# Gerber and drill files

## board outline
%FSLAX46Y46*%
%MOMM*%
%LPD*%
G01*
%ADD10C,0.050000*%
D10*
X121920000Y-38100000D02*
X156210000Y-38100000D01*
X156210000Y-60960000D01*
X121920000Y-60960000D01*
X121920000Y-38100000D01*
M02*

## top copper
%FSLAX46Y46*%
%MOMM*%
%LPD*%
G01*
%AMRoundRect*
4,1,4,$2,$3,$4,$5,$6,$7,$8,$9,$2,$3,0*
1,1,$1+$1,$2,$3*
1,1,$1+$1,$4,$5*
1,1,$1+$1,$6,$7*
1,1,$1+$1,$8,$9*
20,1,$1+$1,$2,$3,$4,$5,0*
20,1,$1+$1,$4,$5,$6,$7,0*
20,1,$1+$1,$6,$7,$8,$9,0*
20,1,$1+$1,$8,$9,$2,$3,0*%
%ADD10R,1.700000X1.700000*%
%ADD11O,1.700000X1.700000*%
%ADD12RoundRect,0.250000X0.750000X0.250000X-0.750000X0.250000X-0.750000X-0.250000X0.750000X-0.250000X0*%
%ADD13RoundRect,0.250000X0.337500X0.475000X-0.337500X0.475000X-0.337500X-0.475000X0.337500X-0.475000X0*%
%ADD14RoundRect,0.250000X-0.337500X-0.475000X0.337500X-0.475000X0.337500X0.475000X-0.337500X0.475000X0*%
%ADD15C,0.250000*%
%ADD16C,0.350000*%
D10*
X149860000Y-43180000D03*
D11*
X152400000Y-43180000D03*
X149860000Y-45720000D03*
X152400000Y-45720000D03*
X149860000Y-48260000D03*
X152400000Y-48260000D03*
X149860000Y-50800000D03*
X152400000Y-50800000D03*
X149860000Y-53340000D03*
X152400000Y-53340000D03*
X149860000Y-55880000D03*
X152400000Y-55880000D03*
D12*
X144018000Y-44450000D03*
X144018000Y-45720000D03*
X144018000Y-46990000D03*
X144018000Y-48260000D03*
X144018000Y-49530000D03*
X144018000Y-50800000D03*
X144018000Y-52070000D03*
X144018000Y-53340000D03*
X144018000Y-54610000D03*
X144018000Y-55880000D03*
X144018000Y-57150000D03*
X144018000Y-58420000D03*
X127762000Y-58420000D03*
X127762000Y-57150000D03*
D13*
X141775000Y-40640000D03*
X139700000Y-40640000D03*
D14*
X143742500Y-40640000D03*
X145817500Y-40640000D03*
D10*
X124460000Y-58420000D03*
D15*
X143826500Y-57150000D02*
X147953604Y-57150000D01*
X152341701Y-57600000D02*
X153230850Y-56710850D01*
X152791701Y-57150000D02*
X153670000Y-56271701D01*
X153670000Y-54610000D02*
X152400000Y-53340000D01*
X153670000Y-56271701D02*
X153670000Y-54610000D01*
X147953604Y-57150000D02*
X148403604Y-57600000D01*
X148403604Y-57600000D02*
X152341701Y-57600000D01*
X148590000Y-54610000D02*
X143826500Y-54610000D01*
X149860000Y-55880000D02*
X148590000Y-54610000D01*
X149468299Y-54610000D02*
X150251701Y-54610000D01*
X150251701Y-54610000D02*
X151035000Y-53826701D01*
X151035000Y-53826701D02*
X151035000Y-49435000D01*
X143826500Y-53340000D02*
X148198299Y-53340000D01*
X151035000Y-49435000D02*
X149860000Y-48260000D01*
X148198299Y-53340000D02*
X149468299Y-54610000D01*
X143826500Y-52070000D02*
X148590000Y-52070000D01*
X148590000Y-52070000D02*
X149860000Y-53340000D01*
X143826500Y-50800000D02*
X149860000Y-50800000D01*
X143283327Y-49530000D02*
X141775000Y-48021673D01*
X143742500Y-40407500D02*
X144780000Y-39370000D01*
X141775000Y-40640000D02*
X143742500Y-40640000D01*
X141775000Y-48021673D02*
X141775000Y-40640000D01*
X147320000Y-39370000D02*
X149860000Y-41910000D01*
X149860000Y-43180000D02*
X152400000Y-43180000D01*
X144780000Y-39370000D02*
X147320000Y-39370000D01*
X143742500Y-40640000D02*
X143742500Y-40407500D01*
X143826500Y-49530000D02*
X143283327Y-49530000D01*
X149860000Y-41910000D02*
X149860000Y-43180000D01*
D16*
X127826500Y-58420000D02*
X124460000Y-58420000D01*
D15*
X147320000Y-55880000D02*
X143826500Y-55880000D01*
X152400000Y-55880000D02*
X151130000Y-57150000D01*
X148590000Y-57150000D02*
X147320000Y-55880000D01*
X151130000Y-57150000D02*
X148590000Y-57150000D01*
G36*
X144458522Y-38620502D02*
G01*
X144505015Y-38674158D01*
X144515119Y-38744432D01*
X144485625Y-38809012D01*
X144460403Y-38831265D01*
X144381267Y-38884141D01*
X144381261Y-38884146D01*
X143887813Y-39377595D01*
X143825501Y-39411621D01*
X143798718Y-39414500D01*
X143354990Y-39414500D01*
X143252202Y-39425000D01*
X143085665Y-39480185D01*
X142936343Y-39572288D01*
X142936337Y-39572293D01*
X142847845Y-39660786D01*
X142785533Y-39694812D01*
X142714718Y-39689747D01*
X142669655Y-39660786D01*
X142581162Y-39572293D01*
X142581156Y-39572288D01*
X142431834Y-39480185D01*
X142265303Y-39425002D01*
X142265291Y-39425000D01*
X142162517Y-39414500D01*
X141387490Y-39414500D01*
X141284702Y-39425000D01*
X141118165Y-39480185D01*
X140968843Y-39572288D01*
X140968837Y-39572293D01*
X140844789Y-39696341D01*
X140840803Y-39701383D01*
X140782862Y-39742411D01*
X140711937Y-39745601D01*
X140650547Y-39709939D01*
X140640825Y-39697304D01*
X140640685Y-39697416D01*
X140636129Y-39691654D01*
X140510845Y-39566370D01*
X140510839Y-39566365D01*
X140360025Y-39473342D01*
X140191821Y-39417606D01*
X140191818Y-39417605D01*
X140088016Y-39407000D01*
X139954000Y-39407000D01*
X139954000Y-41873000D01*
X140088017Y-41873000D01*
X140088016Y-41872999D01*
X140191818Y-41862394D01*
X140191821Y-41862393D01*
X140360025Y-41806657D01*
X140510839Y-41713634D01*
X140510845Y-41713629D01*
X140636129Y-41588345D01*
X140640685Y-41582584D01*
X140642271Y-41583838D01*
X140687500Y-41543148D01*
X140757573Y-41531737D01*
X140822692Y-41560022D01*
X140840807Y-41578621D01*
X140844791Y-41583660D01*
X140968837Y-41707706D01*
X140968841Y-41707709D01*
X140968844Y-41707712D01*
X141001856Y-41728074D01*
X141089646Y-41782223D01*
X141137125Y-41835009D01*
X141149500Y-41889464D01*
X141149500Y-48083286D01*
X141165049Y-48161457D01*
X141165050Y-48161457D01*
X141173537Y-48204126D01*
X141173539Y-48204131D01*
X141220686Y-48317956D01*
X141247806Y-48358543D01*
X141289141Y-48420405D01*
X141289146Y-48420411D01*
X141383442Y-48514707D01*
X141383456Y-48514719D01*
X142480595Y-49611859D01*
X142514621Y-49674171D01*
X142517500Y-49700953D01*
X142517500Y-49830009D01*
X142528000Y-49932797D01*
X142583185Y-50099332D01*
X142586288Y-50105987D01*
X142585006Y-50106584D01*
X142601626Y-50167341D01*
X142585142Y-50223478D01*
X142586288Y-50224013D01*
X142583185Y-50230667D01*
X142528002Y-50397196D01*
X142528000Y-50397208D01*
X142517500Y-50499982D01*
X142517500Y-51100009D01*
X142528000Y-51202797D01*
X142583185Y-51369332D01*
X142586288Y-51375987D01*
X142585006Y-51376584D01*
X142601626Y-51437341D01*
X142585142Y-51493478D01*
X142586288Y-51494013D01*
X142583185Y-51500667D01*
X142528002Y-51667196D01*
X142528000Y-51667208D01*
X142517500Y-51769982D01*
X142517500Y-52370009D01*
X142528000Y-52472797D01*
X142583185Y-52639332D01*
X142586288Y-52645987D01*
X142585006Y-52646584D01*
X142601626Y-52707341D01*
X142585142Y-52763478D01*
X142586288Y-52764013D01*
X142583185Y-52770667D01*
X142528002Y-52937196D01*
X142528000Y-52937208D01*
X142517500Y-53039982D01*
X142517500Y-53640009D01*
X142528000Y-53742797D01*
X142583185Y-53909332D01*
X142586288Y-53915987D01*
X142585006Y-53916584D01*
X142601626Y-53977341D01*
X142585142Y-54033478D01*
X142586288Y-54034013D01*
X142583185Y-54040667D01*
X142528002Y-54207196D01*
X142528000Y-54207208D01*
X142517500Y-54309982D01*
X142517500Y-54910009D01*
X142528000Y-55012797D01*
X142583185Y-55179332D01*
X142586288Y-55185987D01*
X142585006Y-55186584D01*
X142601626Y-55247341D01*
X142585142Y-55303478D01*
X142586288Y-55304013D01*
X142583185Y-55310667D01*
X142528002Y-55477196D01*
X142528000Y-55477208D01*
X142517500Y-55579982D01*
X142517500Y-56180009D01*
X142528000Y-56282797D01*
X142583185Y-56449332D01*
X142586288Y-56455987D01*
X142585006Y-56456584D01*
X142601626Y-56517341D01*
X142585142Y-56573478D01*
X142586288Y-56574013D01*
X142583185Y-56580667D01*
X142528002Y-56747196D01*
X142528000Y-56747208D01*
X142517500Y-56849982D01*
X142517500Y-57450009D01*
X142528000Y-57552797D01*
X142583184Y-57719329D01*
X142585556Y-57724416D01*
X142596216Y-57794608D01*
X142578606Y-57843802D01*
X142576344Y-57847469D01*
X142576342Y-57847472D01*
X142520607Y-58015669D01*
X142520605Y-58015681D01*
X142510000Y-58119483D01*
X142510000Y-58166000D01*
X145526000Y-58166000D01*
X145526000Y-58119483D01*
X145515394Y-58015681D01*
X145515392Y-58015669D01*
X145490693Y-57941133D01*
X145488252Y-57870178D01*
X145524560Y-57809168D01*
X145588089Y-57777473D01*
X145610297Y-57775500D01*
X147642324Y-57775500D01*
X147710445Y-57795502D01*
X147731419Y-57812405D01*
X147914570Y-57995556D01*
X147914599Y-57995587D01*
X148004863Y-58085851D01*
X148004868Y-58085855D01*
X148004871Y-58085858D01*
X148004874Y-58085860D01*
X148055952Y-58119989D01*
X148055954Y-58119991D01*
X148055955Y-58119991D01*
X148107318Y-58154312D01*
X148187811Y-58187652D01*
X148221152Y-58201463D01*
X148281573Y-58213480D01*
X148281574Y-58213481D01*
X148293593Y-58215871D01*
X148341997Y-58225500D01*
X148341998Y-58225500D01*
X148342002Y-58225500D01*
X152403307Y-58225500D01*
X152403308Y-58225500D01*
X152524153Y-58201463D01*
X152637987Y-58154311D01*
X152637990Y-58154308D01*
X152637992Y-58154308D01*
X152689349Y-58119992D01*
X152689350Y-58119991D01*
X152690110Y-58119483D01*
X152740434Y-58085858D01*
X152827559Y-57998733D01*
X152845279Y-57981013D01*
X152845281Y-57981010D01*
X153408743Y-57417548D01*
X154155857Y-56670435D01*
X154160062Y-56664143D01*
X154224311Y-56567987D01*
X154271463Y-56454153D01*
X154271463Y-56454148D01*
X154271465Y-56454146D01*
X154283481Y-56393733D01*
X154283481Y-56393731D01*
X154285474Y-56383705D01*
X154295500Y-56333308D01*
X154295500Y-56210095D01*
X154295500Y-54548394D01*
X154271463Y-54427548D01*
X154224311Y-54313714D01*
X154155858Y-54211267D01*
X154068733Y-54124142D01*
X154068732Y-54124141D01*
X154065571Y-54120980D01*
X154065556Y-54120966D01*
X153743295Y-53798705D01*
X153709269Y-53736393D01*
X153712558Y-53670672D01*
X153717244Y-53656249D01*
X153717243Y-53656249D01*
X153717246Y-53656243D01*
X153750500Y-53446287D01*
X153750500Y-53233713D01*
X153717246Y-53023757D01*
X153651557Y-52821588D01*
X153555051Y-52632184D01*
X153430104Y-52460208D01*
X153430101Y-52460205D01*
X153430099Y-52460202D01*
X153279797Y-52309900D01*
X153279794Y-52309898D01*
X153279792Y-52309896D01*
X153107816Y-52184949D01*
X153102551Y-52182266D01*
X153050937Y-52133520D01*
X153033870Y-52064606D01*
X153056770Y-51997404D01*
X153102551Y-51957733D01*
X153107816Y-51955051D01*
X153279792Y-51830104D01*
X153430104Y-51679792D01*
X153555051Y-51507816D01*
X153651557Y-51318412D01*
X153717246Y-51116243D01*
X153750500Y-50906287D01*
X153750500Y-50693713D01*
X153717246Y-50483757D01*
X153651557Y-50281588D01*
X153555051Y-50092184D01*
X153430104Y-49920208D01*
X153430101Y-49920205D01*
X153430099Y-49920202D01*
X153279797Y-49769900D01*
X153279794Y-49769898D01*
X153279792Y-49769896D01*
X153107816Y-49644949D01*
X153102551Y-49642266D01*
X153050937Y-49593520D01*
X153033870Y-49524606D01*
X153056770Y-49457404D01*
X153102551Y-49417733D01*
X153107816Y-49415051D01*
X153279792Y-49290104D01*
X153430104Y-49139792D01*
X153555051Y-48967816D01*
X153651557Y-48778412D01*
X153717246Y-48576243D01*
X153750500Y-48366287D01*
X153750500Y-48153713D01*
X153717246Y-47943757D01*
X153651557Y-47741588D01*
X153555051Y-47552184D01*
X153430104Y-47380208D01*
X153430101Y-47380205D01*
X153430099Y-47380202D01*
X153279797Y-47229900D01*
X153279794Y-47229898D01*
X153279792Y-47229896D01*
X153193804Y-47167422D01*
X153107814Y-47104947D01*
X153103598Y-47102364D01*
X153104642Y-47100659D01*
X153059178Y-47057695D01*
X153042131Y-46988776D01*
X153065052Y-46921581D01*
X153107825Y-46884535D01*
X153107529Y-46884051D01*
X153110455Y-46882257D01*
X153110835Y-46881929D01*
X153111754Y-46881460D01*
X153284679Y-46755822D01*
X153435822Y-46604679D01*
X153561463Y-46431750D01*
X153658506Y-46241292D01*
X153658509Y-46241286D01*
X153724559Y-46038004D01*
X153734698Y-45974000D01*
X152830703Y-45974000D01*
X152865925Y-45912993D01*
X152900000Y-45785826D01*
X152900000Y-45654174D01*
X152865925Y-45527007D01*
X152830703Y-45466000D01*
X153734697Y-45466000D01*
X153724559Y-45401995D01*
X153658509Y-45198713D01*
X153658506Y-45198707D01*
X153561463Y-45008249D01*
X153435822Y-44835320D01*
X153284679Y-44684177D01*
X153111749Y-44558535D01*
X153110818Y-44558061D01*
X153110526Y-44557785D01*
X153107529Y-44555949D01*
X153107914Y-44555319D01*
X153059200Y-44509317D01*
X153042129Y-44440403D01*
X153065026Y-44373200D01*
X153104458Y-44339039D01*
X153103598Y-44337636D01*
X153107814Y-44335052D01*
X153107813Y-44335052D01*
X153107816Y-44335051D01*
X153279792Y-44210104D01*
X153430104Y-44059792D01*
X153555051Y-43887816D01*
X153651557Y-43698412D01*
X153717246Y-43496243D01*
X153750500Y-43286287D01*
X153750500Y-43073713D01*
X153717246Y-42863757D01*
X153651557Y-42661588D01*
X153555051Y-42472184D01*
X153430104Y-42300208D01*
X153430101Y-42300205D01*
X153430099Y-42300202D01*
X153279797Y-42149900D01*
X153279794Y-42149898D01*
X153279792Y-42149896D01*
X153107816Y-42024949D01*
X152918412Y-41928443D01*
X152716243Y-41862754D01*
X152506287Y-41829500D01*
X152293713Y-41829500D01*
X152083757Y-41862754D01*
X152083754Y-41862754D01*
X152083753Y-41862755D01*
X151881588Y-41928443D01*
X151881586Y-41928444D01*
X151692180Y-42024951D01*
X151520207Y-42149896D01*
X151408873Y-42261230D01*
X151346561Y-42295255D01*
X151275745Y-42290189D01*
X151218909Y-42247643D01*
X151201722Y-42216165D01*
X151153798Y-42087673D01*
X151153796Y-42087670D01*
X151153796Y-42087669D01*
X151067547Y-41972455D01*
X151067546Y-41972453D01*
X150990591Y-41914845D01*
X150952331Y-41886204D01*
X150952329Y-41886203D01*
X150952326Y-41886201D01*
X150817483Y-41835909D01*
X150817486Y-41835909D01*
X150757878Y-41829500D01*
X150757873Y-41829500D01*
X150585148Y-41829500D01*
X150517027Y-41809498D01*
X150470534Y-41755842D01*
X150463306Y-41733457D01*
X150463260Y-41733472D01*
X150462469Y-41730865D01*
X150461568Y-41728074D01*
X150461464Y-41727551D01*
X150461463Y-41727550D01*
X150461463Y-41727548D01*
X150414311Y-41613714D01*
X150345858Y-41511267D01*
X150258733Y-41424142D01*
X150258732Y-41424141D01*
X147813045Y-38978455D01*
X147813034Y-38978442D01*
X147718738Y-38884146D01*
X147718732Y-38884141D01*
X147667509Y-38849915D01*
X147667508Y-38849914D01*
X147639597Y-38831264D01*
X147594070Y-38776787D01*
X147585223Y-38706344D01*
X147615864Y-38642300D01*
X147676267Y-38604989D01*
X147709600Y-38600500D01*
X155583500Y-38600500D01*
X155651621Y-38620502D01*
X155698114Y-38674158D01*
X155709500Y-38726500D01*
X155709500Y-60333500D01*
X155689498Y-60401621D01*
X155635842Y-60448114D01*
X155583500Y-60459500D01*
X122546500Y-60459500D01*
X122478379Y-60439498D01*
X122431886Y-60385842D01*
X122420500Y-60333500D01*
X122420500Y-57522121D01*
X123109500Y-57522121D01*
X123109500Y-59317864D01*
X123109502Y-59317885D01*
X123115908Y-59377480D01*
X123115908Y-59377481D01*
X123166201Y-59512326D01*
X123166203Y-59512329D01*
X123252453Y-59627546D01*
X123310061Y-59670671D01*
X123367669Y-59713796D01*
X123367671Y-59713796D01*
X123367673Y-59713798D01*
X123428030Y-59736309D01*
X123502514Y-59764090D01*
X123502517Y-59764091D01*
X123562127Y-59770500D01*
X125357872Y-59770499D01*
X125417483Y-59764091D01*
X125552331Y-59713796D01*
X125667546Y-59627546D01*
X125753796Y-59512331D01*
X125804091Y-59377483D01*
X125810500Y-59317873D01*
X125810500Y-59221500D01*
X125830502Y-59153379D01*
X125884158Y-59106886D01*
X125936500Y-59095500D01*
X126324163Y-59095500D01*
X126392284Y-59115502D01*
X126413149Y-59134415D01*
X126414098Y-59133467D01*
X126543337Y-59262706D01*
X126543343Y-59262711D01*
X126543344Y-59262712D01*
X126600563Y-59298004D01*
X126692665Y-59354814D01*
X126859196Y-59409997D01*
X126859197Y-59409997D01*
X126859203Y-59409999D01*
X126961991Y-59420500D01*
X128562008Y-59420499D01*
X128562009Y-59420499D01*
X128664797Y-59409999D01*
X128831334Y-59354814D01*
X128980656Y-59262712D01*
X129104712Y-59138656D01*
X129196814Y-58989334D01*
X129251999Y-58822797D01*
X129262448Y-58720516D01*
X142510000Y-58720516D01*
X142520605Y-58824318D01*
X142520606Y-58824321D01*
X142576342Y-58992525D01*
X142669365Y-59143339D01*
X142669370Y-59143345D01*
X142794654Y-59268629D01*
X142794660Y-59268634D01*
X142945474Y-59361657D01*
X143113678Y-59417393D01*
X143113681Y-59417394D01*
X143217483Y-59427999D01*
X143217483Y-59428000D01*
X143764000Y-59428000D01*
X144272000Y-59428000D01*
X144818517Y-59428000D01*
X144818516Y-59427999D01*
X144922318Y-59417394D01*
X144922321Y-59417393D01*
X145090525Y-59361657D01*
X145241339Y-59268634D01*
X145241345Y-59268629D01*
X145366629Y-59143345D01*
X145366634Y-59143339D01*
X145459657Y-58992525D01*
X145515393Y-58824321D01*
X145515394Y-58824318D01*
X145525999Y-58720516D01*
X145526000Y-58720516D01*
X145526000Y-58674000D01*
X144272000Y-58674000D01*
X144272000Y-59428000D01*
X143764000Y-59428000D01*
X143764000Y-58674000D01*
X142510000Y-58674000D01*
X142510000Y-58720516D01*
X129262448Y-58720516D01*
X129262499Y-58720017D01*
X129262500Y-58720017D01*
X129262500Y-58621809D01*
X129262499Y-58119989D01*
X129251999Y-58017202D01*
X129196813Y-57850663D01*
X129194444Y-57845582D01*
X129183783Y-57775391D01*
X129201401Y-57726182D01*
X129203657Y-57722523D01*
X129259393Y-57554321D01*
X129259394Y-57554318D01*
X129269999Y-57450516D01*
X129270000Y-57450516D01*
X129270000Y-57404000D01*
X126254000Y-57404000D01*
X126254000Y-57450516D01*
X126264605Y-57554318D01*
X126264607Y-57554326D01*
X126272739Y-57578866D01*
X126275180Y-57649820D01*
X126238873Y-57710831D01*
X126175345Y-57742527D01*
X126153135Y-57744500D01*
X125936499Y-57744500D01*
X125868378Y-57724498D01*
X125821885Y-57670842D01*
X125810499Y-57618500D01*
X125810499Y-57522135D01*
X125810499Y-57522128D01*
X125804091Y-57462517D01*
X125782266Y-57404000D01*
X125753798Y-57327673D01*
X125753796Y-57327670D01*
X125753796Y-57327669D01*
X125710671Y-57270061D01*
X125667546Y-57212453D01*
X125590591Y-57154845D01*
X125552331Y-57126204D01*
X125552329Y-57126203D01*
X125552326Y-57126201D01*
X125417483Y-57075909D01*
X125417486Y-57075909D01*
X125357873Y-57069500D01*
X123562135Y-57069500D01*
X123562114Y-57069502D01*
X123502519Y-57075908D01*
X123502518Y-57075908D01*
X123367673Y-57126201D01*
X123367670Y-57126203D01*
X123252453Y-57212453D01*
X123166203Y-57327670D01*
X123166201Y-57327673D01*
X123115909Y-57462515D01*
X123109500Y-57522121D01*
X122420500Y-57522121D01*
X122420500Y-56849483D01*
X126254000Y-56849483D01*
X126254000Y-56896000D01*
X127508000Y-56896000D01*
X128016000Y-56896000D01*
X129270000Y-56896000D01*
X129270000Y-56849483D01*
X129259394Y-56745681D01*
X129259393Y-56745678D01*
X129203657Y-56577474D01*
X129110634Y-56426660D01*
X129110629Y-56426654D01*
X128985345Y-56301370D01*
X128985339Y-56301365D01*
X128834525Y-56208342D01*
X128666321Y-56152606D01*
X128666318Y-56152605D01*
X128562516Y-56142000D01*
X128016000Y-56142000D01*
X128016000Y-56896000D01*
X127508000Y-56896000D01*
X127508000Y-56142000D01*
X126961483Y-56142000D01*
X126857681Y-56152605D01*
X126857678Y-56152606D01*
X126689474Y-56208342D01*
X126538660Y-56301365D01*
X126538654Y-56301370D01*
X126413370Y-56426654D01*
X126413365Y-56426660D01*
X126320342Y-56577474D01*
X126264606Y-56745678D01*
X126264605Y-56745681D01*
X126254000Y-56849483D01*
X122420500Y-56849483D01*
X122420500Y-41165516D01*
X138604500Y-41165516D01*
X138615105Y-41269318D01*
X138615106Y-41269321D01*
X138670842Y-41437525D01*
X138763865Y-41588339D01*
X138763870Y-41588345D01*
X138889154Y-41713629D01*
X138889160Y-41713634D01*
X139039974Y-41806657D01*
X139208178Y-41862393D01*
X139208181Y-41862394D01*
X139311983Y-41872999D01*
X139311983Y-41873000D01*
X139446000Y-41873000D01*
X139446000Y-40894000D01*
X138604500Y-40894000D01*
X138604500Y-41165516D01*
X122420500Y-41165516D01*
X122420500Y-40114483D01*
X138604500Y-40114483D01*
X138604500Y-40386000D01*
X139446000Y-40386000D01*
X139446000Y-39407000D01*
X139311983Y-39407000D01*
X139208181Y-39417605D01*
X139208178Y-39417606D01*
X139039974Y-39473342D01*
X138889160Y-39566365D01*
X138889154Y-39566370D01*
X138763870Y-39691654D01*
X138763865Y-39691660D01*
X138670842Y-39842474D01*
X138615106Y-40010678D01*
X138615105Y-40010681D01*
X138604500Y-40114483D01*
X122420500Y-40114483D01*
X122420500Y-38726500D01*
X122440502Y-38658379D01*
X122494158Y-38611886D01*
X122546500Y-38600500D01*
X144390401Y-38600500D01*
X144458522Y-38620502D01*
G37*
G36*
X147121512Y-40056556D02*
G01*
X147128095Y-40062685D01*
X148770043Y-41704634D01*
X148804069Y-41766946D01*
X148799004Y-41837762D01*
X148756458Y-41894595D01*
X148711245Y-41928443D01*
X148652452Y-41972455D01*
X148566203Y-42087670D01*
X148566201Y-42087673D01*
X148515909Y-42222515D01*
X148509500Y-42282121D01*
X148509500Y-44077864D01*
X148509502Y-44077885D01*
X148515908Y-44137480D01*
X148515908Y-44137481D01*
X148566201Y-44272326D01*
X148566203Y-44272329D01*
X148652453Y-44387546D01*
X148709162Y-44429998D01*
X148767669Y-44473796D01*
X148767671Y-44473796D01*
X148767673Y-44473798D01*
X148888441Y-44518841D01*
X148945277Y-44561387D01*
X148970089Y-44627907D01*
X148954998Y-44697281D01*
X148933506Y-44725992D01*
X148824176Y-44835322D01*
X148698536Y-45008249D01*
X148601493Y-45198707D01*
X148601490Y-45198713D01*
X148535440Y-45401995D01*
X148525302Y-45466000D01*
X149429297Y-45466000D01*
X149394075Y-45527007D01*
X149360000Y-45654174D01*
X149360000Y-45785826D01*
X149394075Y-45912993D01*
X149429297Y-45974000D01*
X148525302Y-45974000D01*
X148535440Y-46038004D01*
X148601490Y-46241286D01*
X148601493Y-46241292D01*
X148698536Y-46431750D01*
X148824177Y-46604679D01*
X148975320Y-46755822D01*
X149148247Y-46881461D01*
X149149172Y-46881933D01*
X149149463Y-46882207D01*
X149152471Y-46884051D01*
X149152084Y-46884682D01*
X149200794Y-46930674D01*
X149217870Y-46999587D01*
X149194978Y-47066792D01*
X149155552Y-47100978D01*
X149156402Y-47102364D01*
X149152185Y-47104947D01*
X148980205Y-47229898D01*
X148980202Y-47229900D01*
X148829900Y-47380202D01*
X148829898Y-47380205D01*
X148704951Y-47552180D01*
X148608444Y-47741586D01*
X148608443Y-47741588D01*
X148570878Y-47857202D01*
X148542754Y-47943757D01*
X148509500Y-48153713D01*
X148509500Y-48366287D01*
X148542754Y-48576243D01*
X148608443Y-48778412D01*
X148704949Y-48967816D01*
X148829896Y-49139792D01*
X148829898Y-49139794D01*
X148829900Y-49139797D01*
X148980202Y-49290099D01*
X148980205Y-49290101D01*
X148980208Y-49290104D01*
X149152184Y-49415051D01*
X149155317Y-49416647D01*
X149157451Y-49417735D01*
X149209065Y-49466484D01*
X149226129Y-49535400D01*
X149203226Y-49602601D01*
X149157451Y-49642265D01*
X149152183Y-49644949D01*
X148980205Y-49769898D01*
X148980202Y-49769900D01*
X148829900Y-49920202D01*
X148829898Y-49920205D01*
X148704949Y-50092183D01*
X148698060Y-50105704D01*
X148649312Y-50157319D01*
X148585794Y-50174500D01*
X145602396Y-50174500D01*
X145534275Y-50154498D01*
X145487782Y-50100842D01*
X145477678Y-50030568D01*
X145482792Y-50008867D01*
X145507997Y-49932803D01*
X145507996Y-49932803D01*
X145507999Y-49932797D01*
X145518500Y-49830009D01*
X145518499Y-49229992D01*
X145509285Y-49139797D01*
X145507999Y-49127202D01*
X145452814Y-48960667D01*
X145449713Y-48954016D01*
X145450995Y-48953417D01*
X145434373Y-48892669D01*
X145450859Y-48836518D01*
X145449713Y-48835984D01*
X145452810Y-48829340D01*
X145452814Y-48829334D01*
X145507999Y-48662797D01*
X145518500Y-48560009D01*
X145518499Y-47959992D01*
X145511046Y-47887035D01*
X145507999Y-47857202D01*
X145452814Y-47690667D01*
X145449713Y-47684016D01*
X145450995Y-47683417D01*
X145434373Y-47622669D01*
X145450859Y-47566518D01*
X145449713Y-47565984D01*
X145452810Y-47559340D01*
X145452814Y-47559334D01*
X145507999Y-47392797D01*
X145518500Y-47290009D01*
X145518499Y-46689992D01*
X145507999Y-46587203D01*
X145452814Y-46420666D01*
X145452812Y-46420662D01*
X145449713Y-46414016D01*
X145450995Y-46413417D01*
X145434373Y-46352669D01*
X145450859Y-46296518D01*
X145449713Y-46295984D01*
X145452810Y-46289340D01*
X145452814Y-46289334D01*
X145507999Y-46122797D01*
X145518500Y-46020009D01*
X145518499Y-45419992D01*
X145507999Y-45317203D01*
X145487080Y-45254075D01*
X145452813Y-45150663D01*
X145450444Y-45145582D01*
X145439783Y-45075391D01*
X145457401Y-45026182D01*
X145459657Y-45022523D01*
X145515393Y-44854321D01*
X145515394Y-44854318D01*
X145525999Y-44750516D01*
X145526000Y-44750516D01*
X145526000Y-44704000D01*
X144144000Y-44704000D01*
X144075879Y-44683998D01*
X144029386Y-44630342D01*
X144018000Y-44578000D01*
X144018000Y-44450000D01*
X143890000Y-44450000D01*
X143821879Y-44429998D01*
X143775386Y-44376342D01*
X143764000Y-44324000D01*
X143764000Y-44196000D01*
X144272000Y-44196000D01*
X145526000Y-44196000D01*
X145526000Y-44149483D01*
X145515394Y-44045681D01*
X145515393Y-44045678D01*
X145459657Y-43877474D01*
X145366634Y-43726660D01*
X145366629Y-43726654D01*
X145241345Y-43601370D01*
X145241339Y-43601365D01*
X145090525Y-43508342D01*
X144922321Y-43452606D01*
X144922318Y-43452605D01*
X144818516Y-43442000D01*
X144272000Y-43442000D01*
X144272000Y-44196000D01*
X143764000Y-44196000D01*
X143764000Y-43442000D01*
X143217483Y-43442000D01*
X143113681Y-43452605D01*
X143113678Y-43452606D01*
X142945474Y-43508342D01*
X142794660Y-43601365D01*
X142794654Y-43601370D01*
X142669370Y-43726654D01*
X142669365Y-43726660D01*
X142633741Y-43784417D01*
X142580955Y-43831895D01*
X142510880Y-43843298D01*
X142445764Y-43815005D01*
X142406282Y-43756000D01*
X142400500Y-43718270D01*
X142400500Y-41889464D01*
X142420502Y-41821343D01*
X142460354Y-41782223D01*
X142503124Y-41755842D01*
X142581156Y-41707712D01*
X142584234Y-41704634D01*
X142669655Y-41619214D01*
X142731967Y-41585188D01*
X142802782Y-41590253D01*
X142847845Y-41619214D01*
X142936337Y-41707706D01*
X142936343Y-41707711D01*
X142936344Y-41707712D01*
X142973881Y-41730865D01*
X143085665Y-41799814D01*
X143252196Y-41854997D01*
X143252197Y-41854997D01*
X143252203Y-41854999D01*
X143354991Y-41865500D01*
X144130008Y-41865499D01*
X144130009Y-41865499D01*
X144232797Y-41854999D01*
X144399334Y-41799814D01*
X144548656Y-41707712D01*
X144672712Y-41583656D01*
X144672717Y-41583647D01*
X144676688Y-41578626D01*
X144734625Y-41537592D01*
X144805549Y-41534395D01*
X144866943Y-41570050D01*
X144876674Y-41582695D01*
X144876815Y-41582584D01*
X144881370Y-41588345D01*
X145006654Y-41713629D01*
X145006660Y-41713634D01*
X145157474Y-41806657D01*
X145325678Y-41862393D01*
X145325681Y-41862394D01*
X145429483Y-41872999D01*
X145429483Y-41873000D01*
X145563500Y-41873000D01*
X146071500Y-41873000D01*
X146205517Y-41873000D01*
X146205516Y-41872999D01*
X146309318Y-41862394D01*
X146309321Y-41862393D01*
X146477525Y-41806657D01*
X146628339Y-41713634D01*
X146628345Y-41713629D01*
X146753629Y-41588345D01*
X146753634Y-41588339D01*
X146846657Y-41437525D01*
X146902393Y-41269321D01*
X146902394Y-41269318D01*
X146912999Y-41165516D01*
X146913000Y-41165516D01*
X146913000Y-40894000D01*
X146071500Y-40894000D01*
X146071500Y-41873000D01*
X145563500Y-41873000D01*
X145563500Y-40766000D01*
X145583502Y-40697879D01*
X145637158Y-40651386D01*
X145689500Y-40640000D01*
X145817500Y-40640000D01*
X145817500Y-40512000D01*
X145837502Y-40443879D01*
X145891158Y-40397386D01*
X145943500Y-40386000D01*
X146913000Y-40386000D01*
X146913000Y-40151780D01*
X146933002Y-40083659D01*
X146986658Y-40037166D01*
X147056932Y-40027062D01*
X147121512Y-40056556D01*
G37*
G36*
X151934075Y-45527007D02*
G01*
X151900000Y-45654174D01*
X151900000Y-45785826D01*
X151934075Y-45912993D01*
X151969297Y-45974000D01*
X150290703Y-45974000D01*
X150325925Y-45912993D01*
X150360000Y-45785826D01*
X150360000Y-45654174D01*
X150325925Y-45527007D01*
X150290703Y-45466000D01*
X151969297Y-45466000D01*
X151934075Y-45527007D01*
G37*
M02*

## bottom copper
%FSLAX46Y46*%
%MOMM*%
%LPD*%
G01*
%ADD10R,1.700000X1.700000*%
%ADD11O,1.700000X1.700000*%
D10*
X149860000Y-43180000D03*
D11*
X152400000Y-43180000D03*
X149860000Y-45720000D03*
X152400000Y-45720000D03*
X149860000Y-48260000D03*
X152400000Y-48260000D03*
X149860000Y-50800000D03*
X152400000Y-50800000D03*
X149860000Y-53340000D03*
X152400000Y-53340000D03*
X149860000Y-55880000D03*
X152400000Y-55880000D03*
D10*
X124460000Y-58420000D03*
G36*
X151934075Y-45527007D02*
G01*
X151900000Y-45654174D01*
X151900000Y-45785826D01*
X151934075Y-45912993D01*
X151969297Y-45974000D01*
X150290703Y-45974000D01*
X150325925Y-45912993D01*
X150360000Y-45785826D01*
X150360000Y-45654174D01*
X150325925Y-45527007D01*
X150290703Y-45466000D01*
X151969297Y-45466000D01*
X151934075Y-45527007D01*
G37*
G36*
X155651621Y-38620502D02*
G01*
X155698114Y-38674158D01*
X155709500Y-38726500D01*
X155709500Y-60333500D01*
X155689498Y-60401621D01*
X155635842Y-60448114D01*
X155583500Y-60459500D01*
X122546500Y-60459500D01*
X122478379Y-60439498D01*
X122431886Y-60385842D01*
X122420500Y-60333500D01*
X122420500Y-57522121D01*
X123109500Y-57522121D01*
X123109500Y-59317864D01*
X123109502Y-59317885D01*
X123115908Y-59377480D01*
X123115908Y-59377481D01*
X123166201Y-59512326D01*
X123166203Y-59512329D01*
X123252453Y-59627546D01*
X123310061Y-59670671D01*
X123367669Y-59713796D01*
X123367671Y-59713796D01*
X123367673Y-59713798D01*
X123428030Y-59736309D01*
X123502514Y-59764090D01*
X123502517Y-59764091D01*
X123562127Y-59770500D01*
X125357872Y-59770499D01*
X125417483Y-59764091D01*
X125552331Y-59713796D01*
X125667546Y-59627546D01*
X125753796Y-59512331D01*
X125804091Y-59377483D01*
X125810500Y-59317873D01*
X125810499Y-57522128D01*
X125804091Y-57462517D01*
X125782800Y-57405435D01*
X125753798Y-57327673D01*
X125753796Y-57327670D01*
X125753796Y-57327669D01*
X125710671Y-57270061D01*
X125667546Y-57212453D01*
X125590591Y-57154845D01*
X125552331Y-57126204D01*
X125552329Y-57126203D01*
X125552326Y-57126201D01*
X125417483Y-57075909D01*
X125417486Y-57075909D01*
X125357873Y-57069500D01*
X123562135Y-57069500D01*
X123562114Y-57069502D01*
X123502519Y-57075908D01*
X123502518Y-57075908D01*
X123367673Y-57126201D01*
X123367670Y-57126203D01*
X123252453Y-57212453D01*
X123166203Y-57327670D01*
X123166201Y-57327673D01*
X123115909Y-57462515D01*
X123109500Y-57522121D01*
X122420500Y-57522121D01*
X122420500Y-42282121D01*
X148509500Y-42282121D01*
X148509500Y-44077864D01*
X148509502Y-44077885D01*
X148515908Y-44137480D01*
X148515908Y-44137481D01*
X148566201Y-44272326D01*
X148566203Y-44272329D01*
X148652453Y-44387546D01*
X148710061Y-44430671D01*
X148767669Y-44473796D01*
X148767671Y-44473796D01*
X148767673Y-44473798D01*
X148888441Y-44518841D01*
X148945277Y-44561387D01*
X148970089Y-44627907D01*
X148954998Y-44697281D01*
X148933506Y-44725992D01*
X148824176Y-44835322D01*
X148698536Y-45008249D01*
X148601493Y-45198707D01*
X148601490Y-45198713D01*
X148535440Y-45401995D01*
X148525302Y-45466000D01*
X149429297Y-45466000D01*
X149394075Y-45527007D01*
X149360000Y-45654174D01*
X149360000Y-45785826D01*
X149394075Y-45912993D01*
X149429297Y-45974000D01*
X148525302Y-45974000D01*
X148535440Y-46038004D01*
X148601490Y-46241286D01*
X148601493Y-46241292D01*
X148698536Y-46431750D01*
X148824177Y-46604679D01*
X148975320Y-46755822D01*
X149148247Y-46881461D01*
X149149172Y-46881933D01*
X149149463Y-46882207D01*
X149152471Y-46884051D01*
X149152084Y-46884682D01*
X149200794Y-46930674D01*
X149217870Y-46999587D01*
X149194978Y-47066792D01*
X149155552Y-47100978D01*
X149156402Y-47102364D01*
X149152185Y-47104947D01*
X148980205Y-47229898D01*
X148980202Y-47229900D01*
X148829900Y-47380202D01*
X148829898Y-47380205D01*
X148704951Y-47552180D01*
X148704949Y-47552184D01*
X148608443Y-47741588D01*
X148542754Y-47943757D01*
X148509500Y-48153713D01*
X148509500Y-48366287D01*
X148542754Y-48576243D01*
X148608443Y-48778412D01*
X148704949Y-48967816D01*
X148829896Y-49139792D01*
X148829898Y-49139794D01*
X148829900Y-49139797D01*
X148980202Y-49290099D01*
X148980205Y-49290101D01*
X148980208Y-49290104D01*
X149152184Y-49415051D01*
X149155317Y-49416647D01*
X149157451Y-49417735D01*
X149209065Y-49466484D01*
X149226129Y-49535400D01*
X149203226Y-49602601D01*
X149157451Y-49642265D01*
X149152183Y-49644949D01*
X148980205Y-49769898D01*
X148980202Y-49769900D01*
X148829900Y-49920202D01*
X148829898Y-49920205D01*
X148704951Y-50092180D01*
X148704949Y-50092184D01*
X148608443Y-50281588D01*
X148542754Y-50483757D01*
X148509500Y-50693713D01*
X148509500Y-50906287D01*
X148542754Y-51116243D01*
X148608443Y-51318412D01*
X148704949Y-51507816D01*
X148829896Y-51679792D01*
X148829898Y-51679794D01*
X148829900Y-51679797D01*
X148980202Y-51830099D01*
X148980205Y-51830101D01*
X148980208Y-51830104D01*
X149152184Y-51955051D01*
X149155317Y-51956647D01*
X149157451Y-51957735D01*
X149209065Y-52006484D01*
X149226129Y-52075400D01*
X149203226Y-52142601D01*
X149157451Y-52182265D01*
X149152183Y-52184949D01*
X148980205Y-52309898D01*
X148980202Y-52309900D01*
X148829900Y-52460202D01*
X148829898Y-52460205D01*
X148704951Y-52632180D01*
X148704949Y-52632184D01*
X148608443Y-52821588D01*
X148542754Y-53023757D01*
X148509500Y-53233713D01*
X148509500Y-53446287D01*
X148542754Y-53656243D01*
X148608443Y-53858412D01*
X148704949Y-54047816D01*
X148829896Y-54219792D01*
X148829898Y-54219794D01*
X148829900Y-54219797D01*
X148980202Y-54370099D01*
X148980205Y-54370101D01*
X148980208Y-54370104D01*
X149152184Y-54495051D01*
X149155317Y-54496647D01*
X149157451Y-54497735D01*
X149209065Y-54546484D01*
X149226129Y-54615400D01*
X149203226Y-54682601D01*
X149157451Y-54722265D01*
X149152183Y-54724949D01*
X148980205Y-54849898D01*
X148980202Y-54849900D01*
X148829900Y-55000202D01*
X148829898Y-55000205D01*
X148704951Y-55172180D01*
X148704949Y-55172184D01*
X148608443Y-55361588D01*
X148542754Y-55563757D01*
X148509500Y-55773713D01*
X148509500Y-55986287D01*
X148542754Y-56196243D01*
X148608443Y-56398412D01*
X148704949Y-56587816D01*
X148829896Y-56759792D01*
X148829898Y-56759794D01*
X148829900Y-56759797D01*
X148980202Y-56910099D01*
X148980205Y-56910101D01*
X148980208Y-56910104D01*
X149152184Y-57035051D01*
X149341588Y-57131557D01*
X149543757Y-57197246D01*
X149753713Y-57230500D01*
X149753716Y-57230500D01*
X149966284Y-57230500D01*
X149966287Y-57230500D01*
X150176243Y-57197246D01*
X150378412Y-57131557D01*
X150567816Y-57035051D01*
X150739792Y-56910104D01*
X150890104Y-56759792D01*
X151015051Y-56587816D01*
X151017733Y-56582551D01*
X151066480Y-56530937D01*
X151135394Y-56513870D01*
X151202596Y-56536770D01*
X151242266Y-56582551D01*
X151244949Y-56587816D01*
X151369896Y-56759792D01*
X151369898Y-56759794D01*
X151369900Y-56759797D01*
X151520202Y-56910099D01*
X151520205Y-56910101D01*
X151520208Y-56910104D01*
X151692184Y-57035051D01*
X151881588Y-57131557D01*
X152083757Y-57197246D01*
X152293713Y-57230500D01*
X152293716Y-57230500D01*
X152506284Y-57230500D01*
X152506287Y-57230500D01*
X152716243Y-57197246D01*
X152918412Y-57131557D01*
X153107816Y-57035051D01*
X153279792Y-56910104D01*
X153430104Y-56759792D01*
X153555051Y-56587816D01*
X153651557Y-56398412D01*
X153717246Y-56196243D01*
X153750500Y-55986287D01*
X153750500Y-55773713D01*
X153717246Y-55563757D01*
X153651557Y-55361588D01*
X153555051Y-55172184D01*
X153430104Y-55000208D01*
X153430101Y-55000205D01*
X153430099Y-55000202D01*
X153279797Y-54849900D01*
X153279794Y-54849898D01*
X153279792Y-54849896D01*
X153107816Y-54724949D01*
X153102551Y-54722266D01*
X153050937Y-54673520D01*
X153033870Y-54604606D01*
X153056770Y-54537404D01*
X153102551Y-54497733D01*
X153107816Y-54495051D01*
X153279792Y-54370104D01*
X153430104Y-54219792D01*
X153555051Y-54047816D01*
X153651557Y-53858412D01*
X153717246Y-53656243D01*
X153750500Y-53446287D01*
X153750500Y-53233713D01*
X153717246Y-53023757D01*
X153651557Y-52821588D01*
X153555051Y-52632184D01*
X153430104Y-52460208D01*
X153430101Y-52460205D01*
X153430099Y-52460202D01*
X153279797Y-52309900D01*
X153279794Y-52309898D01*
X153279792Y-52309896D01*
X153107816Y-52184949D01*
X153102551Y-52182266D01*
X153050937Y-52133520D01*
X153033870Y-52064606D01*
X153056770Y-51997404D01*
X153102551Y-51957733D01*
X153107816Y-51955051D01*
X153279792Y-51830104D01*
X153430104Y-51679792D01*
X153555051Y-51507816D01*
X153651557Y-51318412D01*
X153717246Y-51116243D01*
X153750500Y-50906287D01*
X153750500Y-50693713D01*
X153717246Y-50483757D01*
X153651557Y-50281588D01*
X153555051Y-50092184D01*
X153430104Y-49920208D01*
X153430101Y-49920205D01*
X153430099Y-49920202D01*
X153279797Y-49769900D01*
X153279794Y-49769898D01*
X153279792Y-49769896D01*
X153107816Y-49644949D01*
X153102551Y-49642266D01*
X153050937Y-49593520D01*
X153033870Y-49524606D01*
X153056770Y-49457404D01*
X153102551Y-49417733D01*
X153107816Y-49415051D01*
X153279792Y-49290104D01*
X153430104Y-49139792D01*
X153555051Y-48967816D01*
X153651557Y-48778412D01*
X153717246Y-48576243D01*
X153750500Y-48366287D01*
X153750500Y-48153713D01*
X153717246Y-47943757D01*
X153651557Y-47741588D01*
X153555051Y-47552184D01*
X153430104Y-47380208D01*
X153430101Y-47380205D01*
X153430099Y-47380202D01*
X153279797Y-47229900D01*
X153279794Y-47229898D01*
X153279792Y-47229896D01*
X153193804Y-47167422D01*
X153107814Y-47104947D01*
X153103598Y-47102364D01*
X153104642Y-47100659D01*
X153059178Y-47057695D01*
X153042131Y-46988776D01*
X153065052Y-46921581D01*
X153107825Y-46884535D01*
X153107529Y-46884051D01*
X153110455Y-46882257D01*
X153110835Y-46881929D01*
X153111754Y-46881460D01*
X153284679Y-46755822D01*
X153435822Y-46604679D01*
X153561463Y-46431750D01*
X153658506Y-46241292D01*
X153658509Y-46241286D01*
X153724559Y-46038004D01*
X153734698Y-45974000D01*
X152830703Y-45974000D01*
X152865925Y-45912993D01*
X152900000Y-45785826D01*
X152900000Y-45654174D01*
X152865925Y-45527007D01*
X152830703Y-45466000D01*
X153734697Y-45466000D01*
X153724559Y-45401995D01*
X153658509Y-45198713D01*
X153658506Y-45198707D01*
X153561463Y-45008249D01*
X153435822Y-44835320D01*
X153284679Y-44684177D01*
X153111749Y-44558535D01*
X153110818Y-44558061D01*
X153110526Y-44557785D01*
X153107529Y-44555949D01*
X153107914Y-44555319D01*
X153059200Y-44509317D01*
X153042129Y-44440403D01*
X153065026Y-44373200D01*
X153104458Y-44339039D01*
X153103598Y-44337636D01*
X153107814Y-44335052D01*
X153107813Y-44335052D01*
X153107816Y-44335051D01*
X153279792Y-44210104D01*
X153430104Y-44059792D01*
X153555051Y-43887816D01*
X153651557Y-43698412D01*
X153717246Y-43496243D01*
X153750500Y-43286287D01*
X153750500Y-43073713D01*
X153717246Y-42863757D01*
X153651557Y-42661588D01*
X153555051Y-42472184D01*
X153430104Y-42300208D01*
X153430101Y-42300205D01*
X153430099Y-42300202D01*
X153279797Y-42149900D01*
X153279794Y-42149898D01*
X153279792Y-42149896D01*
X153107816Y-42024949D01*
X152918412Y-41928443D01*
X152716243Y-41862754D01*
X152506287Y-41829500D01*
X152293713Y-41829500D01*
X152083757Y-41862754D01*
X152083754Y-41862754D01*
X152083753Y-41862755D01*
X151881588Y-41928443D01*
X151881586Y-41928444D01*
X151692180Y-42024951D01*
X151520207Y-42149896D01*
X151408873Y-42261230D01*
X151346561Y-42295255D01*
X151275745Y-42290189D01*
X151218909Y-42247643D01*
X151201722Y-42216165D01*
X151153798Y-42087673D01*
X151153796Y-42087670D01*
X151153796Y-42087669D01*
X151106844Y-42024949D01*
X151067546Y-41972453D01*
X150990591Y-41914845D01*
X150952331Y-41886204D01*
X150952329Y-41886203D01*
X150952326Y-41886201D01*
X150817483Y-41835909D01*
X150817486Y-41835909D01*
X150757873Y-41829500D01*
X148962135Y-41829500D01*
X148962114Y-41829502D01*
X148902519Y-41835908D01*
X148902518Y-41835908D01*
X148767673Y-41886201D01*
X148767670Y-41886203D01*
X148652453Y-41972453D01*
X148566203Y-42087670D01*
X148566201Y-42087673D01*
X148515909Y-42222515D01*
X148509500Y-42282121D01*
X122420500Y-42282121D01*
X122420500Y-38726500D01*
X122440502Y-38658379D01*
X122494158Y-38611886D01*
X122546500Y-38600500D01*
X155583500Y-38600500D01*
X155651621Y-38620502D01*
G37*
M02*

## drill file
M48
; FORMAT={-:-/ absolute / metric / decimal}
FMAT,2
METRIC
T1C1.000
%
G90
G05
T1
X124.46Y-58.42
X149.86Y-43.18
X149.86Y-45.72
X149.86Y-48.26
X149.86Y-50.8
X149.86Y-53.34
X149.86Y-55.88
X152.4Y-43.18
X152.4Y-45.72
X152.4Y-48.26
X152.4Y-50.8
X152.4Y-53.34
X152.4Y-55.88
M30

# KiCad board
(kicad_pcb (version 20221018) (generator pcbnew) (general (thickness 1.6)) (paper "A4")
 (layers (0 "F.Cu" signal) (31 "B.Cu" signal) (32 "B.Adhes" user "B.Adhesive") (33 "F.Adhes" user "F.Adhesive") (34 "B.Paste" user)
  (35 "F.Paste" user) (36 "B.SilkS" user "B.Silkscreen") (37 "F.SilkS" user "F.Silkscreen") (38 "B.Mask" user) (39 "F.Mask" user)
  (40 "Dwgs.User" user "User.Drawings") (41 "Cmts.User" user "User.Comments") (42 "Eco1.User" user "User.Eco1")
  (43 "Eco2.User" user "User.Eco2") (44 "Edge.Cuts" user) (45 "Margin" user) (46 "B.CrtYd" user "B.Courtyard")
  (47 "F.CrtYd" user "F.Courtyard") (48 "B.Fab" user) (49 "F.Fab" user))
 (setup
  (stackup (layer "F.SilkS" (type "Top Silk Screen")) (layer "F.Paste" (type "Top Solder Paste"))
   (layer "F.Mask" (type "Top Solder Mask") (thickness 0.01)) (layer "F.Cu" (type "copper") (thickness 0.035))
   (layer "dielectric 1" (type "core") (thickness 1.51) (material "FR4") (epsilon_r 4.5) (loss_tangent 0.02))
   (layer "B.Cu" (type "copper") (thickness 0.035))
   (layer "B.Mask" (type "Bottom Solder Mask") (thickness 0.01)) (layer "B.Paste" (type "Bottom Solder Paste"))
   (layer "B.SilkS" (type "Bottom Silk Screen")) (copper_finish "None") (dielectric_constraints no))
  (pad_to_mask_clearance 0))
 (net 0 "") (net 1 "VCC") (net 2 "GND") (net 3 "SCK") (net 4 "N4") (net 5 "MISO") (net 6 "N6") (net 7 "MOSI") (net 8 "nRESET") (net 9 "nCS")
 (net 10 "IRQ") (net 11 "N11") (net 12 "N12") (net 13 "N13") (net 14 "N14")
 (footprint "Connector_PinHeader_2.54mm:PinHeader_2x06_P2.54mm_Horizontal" (layer "F.Cu") (at 149.86 43.18)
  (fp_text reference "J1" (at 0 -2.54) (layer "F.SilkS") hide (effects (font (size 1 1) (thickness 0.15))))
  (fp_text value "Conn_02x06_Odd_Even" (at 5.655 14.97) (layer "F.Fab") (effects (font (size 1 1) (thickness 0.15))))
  (pad "1" thru_hole rect (at 0 0) (size 1.7 1.7) (drill 1) (layers "*.Cu" "*.Mask") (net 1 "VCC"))
  (pad "2" thru_hole oval (at 2.54 0) (size 1.7 1.7) (drill 1) (layers "*.Cu" "*.Mask") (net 1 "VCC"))
  (pad "3" thru_hole oval (at 0 2.54) (size 1.7 1.7) (drill 1) (layers "*.Cu" "*.Mask") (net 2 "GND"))
  (pad "4" thru_hole oval (at 2.54 2.54) (size 1.7 1.7) (drill 1) (layers "*.Cu" "*.Mask") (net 2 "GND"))
  (pad "5" thru_hole oval (at 0 5.08) (size 1.7 1.7) (drill 1) (layers "*.Cu" "*.Mask") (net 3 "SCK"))
  (pad "6" thru_hole oval (at 2.54 5.08) (size 1.7 1.7) (drill 1) (layers "*.Cu" "*.Mask") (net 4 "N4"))
  (pad "7" thru_hole oval (at 0 7.62) (size 1.7 1.7) (drill 1) (layers "*.Cu" "*.Mask") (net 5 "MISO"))
  (pad "8" thru_hole oval (at 2.54 7.62) (size 1.7 1.7) (drill 1) (layers "*.Cu" "*.Mask") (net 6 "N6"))
  (pad "9" thru_hole oval (at 0 10.16) (size 1.7 1.7) (drill 1) (layers "*.Cu" "*.Mask") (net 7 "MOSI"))
  (pad "10" thru_hole oval (at 2.54 10.16) (size 1.7 1.7) (drill 1) (layers "*.Cu" "*.Mask") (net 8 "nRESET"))
  (pad "11" thru_hole oval (at 0 12.7) (size 1.7 1.7) (drill 1) (layers "*.Cu" "*.Mask") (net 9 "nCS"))
  (pad "12" thru_hole oval (at 2.54 12.7) (size 1.7 1.7) (drill 1) (layers "*.Cu" "*.Mask") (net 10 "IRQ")))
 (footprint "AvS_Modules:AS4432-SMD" (layer "F.Cu") (at 135.89 52.07 180)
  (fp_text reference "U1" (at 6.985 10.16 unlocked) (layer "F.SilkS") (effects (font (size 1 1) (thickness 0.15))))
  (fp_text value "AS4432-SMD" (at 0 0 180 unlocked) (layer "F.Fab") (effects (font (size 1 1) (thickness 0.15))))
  (pad "1" smd roundrect (at -8.128 7.62 180) (size 2 1) (layers "F.Cu" "F.Paste" "F.Mask") (roundrect_rratio 0.25) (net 2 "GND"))
  (pad "2" smd roundrect (at -8.128 6.35 180) (size 2 1) (layers "F.Cu" "F.Paste" "F.Mask") (roundrect_rratio 0.25) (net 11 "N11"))
  (pad "3" smd roundrect (at -8.128 5.08 180) (size 2 1) (layers "F.Cu" "F.Paste" "F.Mask") (roundrect_rratio 0.25) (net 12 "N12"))
  (pad "4" smd roundrect (at -8.128 3.81 180) (size 2 1) (layers "F.Cu" "F.Paste" "F.Mask") (roundrect_rratio 0.25) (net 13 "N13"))
  (pad "5" smd roundrect (at -8.128 2.54 180) (size 2 1) (layers "F.Cu" "F.Paste" "F.Mask") (roundrect_rratio 0.25) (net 1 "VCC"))
  (pad "6" smd roundrect (at -8.128 1.27 180) (size 2 1) (layers "F.Cu" "F.Paste" "F.Mask") (roundrect_rratio 0.25) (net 5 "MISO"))
  (pad "7" smd roundrect (at -8.128 0 180) (size 2 1) (layers "F.Cu" "F.Paste" "F.Mask") (roundrect_rratio 0.25) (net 7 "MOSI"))
  (pad "8" smd roundrect (at -8.128 -1.27 180) (size 2 1) (layers "F.Cu" "F.Paste" "F.Mask") (roundrect_rratio 0.25) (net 3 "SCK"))
  (pad "9" smd roundrect (at -8.128 -2.54 180) (size 2 1) (layers "F.Cu" "F.Paste" "F.Mask") (roundrect_rratio 0.25) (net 9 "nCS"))
  (pad "10" smd roundrect (at -8.128 -3.81 180) (size 2 1) (layers "F.Cu" "F.Paste" "F.Mask") (roundrect_rratio 0.25) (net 10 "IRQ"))
  (pad "11" smd roundrect (at -8.128 -5.08 180) (size 2 1) (layers "F.Cu" "F.Paste" "F.Mask") (roundrect_rratio 0.25) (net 8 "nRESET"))
  (pad "12" smd roundrect (at -8.128 -6.35 180) (size 2 1) (layers "F.Cu" "F.Paste" "F.Mask") (roundrect_rratio 0.25) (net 2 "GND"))
  (pad "13" smd roundrect (at 8.128 -6.35 180) (size 2 1) (layers "F.Cu" "F.Paste" "F.Mask") (roundrect_rratio 0.25) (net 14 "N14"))
  (pad "14" smd roundrect (at 8.128 -5.08 180) (size 2 1) (layers "F.Cu" "F.Paste" "F.Mask") (roundrect_rratio 0.25) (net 2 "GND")))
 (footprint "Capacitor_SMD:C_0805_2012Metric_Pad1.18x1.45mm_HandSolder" (layer "F.Cu") (at 140.7375 40.64 180)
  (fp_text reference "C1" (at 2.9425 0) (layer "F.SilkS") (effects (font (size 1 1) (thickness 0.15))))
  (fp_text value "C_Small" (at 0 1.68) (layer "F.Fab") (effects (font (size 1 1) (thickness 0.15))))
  (pad "1" smd roundrect (at -1.0375 0 180) (size 1.175 1.45) (layers "F.Cu" "F.Paste" "F.Mask") (roundrect_rratio 0.2127659574)
   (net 1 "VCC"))
  (pad "2" smd roundrect (at 1.0375 0 180) (size 1.175 1.45) (layers "F.Cu" "F.Paste" "F.Mask") (roundrect_rratio 0.2127659574)
   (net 2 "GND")))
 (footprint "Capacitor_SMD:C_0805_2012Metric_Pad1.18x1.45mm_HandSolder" (layer "F.Cu") (at 144.78 40.64)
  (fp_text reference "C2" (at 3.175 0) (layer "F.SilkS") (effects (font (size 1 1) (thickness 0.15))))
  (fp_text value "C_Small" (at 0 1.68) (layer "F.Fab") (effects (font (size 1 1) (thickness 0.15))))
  (pad "1" smd roundrect (at -1.0375 0) (size 1.175 1.45) (layers "F.Cu" "F.Paste" "F.Mask") (roundrect_rratio 0.2127659574) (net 1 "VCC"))
  (pad "2" smd roundrect (at 1.0375 0) (size 1.175 1.45) (layers "F.Cu" "F.Paste" "F.Mask") (roundrect_rratio 0.2127659574) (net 2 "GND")))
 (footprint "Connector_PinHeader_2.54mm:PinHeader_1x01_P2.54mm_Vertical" (layer "F.Cu") (at 124.46 58.42)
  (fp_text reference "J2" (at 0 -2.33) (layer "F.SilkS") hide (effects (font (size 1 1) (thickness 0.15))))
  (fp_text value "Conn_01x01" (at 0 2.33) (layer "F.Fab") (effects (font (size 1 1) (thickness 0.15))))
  (pad "1" thru_hole rect (at 0 0) (size 1.7 1.7) (drill 1) (layers "*.Cu" "*.Mask") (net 14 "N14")))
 (gr_rect (start 121.92 38.1) (end 156.21 60.96) (stroke (width 0.05) (type solid)) (fill none) (layer "Edge.Cuts"))
 (segment (start 143.8265 57.15) (end 147.953604 57.15) (width 0.25) (layer "F.Cu") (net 8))
 (segment (start 152.341701 57.6) (end 153.23085 56.71085) (width 0.25) (layer "F.Cu") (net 8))
 (segment (start 152.791701 57.15) (end 153.67 56.271701) (width 0.25) (layer "F.Cu") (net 8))
 (segment (start 153.67 54.61) (end 152.4 53.34) (width 0.25) (layer "F.Cu") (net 8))
 (segment (start 153.67 56.271701) (end 153.67 54.61) (width 0.25) (layer "F.Cu") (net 8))
 (segment (start 147.953604 57.15) (end 148.403604 57.6) (width 0.25) (layer "F.Cu") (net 8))
 (segment (start 148.403604 57.6) (end 152.341701 57.6) (width 0.25) (layer "F.Cu") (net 8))
 (segment (start 148.59 54.61) (end 143.8265 54.61) (width 0.25) (layer "F.Cu") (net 9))
 (segment (start 149.86 55.88) (end 148.59 54.61) (width 0.25) (layer "F.Cu") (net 9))
 (segment (start 149.468299 54.61) (end 150.251701 54.61) (width 0.25) (layer "F.Cu") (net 3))
 (segment (start 150.251701 54.61) (end 151.035 53.826701) (width 0.25) (layer "F.Cu") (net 3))
 (segment (start 151.035 53.826701) (end 151.035 49.435) (width 0.25) (layer "F.Cu") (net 3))
 (segment (start 143.8265 53.34) (end 148.198299 53.34) (width 0.25) (layer "F.Cu") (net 3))
 (segment (start 151.035 49.435) (end 149.86 48.26) (width 0.25) (layer "F.Cu") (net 3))
 (segment (start 148.198299 53.34) (end 149.468299 54.61) (width 0.25) (layer "F.Cu") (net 3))
 (segment (start 143.8265 52.07) (end 148.59 52.07) (width 0.25) (layer "F.Cu") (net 7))
 (segment (start 148.59 52.07) (end 149.86 53.34) (width 0.25) (layer "F.Cu") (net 7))
 (segment (start 143.8265 50.8) (end 149.86 50.8) (width 0.25) (layer "F.Cu") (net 5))
 (segment (start 143.283327 49.53) (end 141.775 48.021673) (width 0.25) (layer "F.Cu") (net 1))
 (segment (start 143.7425 40.4075) (end 144.78 39.37) (width 0.25) (layer "F.Cu") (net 1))
 (segment (start 141.775 40.64) (end 143.7425 40.64) (width 0.25) (layer "F.Cu") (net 1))
 (segment (start 141.775 48.021673) (end 141.775 40.64) (width 0.25) (layer "F.Cu") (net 1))
 (segment (start 147.32 39.37) (end 149.86 41.91) (width 0.25) (layer "F.Cu") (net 1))
 (segment (start 149.86 43.18) (end 152.4 43.18) (width 0.25) (layer "F.Cu") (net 1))
 (segment (start 144.78 39.37) (end 147.32 39.37) (width 0.25) (layer "F.Cu") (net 1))
 (segment (start 143.7425 40.64) (end 143.7425 40.4075) (width 0.25) (layer "F.Cu") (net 1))
 (segment (start 143.8265 49.53) (end 143.283327 49.53) (width 0.25) (layer "F.Cu") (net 1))
 (segment (start 149.86 41.91) (end 149.86 43.18) (width 0.25) (layer "F.Cu") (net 1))
 (segment (start 127.8265 58.42) (end 124.46 58.42) (width 0.35) (layer "F.Cu") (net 14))
 (segment (start 147.32 55.88) (end 143.8265 55.88) (width 0.25) (layer "F.Cu") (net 10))
 (segment (start 152.4 55.88) (end 151.13 57.15) (width 0.25) (layer "F.Cu") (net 10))
 (segment (start 148.59 57.15) (end 147.32 55.88) (width 0.25) (layer "F.Cu") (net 10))
 (segment (start 151.13 57.15) (end 148.59 57.15) (width 0.25) (layer "F.Cu") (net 10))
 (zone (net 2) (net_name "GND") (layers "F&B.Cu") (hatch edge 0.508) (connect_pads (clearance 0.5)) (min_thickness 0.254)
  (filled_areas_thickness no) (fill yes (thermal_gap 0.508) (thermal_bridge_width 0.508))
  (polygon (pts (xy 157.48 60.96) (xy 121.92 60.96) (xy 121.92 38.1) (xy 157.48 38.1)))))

